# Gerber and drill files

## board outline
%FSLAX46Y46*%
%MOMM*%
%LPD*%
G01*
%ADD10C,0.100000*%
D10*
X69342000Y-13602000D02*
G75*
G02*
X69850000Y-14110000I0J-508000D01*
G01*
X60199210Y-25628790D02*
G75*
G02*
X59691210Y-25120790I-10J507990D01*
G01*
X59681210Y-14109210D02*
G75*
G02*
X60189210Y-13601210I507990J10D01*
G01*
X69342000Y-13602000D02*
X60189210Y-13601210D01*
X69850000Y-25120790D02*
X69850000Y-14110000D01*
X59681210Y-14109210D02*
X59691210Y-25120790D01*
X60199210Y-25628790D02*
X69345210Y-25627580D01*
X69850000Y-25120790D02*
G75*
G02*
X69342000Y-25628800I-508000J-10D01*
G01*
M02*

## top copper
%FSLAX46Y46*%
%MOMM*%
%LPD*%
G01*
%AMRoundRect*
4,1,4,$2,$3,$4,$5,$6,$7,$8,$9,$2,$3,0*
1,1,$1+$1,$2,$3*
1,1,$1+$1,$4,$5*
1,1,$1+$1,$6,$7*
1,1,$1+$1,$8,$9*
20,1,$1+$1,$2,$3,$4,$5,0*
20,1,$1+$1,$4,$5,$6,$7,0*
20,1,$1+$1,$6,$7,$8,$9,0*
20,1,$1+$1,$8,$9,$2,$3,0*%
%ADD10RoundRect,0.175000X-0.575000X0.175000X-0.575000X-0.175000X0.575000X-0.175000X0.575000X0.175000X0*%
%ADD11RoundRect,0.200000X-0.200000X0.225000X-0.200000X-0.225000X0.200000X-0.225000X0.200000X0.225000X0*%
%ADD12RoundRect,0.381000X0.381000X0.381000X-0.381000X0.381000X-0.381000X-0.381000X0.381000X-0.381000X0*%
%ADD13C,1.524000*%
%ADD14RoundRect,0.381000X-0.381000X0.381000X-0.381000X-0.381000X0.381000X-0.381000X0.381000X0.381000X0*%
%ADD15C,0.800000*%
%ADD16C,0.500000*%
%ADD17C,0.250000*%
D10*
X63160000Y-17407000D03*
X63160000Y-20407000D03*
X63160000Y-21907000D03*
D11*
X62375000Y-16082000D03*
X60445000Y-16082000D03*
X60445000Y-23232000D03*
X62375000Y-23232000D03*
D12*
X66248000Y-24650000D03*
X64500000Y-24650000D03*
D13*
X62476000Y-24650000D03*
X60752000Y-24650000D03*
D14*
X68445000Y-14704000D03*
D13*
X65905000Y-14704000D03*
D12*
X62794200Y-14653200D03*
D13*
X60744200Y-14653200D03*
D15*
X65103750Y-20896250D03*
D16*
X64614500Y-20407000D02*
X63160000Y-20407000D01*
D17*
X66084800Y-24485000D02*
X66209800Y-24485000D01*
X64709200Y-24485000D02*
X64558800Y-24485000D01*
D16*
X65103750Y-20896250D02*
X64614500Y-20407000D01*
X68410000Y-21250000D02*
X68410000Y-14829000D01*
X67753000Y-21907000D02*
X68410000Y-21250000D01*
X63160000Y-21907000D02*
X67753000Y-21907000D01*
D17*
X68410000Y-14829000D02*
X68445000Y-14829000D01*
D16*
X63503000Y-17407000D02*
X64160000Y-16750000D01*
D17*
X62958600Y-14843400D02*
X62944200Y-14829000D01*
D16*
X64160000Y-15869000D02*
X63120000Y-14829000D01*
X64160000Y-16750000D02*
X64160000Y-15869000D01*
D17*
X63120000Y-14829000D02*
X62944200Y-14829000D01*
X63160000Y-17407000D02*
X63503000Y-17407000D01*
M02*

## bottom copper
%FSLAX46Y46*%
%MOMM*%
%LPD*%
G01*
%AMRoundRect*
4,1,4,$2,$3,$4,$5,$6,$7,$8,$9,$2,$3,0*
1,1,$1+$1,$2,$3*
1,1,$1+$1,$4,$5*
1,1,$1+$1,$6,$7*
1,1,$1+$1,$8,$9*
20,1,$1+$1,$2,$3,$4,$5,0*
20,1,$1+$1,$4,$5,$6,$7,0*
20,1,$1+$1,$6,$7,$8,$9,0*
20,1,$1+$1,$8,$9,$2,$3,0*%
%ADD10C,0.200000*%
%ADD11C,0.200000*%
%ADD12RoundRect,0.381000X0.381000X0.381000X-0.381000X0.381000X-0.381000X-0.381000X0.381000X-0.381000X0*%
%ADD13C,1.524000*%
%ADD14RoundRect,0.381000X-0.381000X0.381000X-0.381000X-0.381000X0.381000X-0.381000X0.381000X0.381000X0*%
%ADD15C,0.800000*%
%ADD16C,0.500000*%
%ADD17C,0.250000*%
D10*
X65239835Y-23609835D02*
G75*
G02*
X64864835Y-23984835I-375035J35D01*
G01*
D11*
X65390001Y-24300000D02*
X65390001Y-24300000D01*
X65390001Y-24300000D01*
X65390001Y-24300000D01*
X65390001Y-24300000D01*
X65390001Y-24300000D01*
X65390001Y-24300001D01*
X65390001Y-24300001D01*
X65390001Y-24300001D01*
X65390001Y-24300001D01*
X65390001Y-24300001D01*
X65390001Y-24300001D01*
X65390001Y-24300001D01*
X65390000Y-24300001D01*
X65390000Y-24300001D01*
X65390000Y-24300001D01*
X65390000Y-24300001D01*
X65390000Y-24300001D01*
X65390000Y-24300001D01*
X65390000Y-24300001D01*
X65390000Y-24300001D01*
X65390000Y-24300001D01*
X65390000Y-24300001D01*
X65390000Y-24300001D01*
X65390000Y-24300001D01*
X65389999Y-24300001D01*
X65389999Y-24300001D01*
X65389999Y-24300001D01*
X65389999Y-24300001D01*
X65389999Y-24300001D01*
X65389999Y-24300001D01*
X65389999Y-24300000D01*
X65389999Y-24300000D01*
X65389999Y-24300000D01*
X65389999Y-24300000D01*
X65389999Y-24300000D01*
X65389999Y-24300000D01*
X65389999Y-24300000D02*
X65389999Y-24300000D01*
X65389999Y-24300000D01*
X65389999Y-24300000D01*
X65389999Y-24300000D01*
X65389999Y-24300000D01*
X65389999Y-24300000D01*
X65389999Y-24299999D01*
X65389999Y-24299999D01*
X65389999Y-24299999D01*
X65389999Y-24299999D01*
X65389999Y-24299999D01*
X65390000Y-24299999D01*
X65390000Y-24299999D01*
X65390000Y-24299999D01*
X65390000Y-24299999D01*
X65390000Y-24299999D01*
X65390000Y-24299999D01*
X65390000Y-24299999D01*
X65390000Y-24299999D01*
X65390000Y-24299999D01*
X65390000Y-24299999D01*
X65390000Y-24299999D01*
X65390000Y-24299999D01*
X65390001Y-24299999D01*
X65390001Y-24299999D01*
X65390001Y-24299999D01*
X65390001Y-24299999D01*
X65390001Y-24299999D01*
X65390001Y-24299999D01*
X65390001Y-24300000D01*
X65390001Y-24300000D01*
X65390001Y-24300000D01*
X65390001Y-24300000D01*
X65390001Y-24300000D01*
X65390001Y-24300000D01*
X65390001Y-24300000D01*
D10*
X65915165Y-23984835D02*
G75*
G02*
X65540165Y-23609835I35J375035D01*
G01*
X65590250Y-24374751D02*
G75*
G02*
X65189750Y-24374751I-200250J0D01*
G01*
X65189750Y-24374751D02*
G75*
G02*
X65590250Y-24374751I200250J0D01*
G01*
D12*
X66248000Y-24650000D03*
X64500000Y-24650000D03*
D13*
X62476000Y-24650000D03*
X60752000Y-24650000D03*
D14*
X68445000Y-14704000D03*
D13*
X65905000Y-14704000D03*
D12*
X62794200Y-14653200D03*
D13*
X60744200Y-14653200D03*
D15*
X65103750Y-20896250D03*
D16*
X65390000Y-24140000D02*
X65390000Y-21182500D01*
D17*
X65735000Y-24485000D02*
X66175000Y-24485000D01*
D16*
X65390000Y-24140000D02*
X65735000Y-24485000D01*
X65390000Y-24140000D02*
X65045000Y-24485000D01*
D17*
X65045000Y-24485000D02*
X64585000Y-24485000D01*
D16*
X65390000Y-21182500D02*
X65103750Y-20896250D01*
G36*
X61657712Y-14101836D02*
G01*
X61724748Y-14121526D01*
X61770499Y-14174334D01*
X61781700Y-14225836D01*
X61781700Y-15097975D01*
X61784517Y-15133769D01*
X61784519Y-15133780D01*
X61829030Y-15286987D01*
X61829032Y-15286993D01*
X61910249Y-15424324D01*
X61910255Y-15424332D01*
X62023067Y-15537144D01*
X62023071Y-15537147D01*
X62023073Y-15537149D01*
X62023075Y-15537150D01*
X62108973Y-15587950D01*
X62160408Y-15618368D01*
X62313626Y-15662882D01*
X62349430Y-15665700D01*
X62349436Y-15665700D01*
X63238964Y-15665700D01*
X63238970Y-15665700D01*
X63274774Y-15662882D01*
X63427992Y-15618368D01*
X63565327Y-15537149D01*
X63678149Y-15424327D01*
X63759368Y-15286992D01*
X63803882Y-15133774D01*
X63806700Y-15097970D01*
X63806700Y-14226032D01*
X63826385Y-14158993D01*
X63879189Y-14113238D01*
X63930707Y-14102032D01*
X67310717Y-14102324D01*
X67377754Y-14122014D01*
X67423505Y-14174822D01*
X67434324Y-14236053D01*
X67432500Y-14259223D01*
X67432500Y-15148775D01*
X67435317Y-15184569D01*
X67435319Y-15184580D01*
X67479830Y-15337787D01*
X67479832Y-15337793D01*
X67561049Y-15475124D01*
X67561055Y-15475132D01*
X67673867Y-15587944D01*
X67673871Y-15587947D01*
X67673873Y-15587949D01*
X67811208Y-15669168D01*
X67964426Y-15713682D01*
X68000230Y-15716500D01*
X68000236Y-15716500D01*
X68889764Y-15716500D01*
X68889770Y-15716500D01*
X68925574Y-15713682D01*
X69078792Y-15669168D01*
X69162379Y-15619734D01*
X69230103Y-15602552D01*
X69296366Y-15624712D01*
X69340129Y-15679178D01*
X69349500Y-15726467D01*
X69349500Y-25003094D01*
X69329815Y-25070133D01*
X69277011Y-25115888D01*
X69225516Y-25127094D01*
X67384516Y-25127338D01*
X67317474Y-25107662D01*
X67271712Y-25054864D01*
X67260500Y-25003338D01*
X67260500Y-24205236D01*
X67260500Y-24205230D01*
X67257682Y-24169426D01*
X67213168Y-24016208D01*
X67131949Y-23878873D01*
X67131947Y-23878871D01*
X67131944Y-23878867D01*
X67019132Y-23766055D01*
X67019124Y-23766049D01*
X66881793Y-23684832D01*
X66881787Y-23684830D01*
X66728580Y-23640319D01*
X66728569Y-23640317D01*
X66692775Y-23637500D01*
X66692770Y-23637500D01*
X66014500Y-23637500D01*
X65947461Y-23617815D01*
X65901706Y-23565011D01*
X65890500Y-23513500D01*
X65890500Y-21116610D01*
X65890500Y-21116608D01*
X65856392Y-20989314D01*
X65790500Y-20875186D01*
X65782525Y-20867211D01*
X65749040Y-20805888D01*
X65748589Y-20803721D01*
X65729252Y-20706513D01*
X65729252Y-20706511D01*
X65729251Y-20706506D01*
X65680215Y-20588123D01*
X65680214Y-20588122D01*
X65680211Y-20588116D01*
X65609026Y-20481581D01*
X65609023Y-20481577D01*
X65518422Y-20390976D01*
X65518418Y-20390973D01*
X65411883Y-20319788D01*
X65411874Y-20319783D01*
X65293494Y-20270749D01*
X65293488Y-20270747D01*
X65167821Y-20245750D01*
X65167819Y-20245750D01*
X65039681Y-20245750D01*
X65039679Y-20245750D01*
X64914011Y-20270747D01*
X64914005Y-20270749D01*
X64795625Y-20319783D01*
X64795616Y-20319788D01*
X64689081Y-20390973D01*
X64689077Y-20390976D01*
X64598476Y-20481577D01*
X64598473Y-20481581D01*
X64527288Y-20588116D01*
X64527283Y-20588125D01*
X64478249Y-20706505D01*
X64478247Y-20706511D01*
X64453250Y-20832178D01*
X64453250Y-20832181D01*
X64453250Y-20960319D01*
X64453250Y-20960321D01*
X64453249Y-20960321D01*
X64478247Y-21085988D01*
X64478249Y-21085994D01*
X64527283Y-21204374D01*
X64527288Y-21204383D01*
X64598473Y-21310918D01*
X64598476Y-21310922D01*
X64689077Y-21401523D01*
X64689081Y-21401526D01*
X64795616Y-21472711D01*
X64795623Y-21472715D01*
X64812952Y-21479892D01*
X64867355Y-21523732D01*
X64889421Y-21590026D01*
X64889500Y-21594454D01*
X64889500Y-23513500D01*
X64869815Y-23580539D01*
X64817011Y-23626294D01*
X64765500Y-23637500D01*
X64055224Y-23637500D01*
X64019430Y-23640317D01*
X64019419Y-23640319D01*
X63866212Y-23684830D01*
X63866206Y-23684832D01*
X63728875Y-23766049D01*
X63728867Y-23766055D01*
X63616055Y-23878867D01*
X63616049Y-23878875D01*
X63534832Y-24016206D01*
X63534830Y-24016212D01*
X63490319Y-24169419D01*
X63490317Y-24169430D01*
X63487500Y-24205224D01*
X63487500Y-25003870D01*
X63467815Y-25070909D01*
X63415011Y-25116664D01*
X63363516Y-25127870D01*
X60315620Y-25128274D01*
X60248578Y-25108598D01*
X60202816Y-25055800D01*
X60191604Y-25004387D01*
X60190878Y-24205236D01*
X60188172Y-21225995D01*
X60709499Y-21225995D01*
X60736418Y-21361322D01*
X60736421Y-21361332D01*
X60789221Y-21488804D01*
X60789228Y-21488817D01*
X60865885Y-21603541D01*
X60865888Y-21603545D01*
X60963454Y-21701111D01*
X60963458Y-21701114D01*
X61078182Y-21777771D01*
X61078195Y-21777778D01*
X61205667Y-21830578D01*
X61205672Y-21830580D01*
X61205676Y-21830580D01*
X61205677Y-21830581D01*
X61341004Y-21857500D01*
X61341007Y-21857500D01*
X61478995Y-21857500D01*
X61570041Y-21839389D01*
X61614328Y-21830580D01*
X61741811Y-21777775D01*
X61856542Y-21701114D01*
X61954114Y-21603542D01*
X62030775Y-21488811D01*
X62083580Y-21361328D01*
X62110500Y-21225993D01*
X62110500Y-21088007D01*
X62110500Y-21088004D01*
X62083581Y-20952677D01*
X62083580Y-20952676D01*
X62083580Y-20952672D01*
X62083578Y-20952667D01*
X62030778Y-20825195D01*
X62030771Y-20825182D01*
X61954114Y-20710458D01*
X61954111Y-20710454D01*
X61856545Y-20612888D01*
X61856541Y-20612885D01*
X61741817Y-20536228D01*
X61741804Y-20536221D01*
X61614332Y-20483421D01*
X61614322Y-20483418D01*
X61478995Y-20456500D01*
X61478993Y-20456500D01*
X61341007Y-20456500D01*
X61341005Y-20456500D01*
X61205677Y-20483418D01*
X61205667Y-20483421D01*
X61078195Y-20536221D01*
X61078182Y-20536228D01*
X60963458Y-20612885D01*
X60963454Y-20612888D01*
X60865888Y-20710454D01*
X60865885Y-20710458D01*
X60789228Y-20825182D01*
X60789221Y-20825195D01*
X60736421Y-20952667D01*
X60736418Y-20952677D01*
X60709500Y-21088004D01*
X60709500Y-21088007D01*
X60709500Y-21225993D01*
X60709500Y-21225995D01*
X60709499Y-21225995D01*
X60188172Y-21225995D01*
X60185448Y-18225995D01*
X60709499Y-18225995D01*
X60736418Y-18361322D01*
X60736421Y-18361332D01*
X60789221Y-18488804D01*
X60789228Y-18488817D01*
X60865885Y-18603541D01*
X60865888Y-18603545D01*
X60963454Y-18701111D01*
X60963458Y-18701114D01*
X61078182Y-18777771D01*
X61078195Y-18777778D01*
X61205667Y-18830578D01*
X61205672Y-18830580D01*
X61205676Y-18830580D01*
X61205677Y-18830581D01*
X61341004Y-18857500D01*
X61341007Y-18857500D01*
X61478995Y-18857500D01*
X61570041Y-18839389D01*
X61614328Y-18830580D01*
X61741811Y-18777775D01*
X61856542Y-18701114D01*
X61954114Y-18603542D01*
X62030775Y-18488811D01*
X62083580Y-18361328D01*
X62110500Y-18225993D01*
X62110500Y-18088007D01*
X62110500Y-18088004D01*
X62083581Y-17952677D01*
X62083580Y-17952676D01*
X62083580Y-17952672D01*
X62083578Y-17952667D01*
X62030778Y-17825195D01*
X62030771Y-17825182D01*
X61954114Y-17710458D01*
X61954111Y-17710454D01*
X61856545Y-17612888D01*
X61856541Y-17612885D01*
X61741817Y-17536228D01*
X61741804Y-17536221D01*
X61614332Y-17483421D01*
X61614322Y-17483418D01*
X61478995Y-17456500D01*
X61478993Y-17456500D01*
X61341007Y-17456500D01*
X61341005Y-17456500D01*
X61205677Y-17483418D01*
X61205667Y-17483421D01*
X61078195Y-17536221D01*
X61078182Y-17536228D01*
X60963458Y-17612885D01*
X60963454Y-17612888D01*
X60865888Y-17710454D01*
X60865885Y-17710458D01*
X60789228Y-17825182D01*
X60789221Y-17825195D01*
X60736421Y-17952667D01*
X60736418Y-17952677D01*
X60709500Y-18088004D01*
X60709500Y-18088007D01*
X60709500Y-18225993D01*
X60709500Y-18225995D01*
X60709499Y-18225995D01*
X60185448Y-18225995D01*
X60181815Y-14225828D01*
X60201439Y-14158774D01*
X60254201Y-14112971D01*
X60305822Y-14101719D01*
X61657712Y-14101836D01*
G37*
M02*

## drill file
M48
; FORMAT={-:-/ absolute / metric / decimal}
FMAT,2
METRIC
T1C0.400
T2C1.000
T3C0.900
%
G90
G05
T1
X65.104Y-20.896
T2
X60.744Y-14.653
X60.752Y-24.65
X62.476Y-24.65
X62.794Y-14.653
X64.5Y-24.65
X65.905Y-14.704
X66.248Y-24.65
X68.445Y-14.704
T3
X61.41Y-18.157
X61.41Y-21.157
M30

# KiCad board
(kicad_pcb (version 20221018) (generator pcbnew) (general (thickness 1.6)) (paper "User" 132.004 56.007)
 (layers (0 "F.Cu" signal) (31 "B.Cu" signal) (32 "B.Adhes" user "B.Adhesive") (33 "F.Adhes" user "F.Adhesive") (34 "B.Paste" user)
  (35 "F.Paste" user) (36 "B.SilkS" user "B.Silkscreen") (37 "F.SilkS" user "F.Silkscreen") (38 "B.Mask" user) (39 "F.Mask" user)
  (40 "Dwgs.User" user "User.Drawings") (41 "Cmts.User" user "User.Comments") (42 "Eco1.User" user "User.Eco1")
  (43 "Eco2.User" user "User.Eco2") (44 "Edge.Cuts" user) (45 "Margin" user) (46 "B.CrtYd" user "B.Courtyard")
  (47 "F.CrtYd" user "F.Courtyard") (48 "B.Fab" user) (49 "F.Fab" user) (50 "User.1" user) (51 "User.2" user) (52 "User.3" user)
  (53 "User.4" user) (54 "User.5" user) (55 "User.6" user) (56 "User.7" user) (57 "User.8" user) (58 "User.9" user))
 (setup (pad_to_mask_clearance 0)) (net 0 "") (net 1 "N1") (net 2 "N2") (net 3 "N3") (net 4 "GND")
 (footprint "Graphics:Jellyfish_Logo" (layer "F.Cu") (at 68.475 24.4)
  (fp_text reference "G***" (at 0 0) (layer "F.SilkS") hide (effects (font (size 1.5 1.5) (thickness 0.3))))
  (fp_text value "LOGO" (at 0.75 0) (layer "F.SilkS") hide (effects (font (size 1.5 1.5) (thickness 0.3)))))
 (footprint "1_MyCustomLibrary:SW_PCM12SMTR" (layer "F.Cu") (at 61.41 19.657 -90)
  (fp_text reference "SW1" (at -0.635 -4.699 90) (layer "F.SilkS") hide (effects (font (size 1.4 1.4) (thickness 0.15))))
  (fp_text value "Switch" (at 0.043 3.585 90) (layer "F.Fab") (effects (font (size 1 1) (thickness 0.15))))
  (pad "" np_thru_hole circle (at -1.5 0 270) (size 0.9 0.9) (drill 0.9) (layers "*.Cu" "*.Mask"))
  (pad "" np_thru_hole circle (at 1.5 0 270) (size 0.9 0.9) (drill 0.9) (layers "*.Cu" "*.Mask"))
  (pad "1" smd roundrect (at -2.25 -1.75 270) (size 0.7 1.5) (layers "F.Cu" "F.Paste" "F.Mask") (roundrect_rratio 0.25) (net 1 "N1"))
  (pad "2" smd roundrect (at 0.75 -1.75 270) (size 0.7 1.5) (layers "F.Cu" "F.Paste" "F.Mask") (roundrect_rratio 0.25) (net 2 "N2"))
  (pad "3" smd roundrect (at 2.25 -1.75 270) (size 0.7 1.5) (layers "F.Cu" "F.Paste" "F.Mask") (roundrect_rratio 0.25) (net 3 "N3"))
  (pad "S1" smd roundrect (at -3.575 -0.965 270) (size 0.85 0.8) (layers "F.Cu" "F.Paste" "F.Mask") (roundrect_rratio 0.25))
  (pad "S2" smd roundrect (at -3.575 0.965 270) (size 0.85 0.8) (layers "F.Cu" "F.Paste" "F.Mask") (roundrect_rratio 0.25))
  (pad "S3" smd roundrect (at 3.575 0.965 270) (size 0.85 0.8) (layers "F.Cu" "F.Paste" "F.Mask") (roundrect_rratio 0.25))
  (pad "S4" smd roundrect (at 3.575 -0.965 270) (size 0.85 0.8) (layers "F.Cu" "F.Paste" "F.Mask") (roundrect_rratio 0.25)))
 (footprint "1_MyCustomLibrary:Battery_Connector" (layer "F.Cu") (at 64.5 24.65 180)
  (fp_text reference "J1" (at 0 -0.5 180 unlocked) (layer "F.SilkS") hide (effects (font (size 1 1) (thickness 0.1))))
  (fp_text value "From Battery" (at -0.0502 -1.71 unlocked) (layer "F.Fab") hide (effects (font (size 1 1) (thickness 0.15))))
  (pad "1" thru_hole roundrect (at -1.748 0 180) (size 1.524 1.524) (drill oval 1) (layers "*.Cu" "*.Mask") (roundrect_rratio 0.25)
   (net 2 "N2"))
  (pad "1" thru_hole roundrect (at 0 0 180) (size 1.524 1.524) (drill oval 1) (layers "*.Cu" "*.Mask") (roundrect_rratio 0.25) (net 2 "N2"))
  (pad "2" thru_hole circle (at 2.024 0 180) (size 1.524 1.524) (drill 1) (layers "*.Cu" "*.Mask") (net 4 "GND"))
  (pad "2" thru_hole circle (at 3.748 0 180) (size 1.524 1.524) (drill 1) (layers "*.Cu" "*.Mask") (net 4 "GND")))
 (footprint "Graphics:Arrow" (layer "F.Cu") (at 64.8 21.125 180)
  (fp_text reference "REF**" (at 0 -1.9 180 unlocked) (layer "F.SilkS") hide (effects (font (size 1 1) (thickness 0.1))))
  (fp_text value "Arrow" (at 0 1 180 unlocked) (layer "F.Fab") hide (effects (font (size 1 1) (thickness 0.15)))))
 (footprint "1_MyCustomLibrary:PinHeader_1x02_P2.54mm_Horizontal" (layer "F.Cu") (at 68.445 14.704 -90)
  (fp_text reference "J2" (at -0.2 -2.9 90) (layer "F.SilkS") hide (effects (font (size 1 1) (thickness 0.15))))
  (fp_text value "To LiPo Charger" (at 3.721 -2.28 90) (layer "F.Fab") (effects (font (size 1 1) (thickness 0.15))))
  (pad "1" thru_hole roundrect (at 0 0 270) (size 1.524 1.524) (drill 1) (layers "*.Cu" "*.Mask") (roundrect_rratio 0.25) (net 3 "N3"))
  (pad "2" thru_hole circle (at 0 2.54 270) (size 1.524 1.524) (drill 1) (layers "*.Cu" "*.Mask") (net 4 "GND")))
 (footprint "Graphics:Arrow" (layer "F.Cu") (at 64.8 20.615)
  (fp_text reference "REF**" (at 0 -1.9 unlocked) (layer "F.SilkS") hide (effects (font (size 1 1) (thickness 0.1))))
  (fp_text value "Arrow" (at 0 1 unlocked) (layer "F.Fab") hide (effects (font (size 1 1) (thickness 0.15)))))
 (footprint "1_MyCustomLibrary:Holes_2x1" (layer "F.Cu") (at 62.0442 14.6532 180)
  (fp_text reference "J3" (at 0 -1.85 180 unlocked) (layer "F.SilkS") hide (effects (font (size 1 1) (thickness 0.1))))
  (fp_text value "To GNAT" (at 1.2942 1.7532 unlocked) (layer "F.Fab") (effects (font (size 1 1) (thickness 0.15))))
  (pad "1" thru_hole roundrect (at -0.75 0 180) (size 1.524 1.524) (drill 1) (layers "*.Cu" "*.Mask") (roundrect_rratio 0.25) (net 1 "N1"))
  (pad "2" thru_hole circle (at 1.3 0 180) (size 1.524 1.524) (drill 1) (layers "*.Cu" "*.Mask") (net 4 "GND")))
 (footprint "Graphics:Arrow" (layer "B.Cu") (at 60.475 20.05)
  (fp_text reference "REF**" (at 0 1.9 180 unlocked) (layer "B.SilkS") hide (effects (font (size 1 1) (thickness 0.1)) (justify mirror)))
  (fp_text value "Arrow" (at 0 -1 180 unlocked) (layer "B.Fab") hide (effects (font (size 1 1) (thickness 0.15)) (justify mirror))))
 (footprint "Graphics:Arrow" (layer "B.Cu") (at 60.475 19.54 180)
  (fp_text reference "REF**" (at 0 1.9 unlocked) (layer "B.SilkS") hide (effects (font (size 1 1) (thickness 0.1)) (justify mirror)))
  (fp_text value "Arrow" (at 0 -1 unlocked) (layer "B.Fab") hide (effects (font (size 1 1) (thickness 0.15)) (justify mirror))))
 (gr_arc (start 65.239835 23.609835) (mid 65.13 23.875) (end 64.864835 23.984835) (stroke (width 0.2) (type default)) (layer "B.Cu"))
 (gr_circle (center 65.39 24.3) (end 65.39 24.3) (stroke (width 0.2) (type default)) (fill none) (layer "B.Cu"))
 (gr_arc (start 65.915165 23.984835) (mid 65.65 23.875) (end 65.540165 23.609835) (stroke (width 0.2) (type default)) (layer "B.Cu"))
 (gr_circle (center 65.39 24.374751) (end 65.4 24.174751) (stroke (width 0.2) (type default)) (fill none) (layer "B.Cu"))
 (gr_arc (start 69.342 13.602) (mid 69.70121 13.75079) (end 69.85 14.11) (stroke (width 0.1) (type default)) (layer "Edge.Cuts"))
 (gr_arc (start 60.19921 25.62879) (mid 59.84 25.48) (end 59.69121 25.12079) (stroke (width 0.1) (type default)) (layer "Edge.Cuts"))
 (gr_arc (start 59.68121 14.10921) (mid 59.83 13.75) (end 60.18921 13.60121) (stroke (width 0.1) (type default)) (layer "Edge.Cuts"))
 (gr_line (start 69.342 13.602) (end 60.18921 13.60121) (stroke (width 0.1) (type default)) (layer "Edge.Cuts"))
 (gr_line (start 69.85 25.12079) (end 69.85 14.11) (stroke (width 0.1) (type default)) (layer "Edge.Cuts"))
 (gr_line (start 59.68121 14.10921) (end 59.69121 25.12079) (stroke (width 0.1) (type default)) (layer "Edge.Cuts"))
 (gr_line (start 60.19921 25.62879) (end 69.34521 25.62758) (stroke (width 0.1) (type default)) (layer "Edge.Cuts"))
 (gr_arc (start 69.85 25.12079) (mid 69.70121 25.48) (end 69.342 25.62879) (stroke (width 0.1) (type default)) (layer "Edge.Cuts"))
 (segment (start 64.6145 20.407) (end 63.16 20.407) (width 0.5) (layer "F.Cu") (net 2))
 (segment (start 66.0848 24.485) (end 66.2098 24.485) (width 0.25) (layer "F.Cu") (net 2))
 (segment (start 64.7092 24.485) (end 64.5588 24.485) (width 0.25) (layer "F.Cu") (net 2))
 (segment (start 65.10375 20.89625) (end 64.6145 20.407) (width 0.5) (layer "F.Cu") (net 2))
 (via (at 65.10375 20.89625) (size 0.8) (drill 0.4) (layers "F.Cu" "B.Cu") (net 2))
 (segment (start 65.39 24.14) (end 65.39 21.1825) (width 0.5) (layer "B.Cu") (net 2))
 (segment (start 65.735 24.485) (end 66.175 24.485) (width 0.25) (layer "B.Cu") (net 2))
 (segment (start 65.39 24.14) (end 65.735 24.485) (width 0.5) (layer "B.Cu") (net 2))
 (segment (start 65.39 24.14) (end 65.045 24.485) (width 0.5) (layer "B.Cu") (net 2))
 (segment (start 65.045 24.485) (end 64.585 24.485) (width 0.25) (layer "B.Cu") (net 2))
 (segment (start 65.39 21.1825) (end 65.10375 20.89625) (width 0.5) (layer "B.Cu") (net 2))
 (segment (start 68.41 21.25) (end 68.41 14.829) (width 0.5) (layer "F.Cu") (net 3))
 (segment (start 67.753 21.907) (end 68.41 21.25) (width 0.5) (layer "F.Cu") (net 3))
 (segment (start 63.16 21.907) (end 67.753 21.907) (width 0.5) (layer "F.Cu") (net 3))
 (segment (start 68.41 14.829) (end 68.445 14.829) (width 0.25) (layer "F.Cu") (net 3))
 (segment (start 63.503 17.407) (end 64.16 16.75) (width 0.5) (layer "F.Cu") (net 1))
 (segment (start 62.9586 14.8434) (end 62.9442 14.829) (width 0.25) (layer "F.Cu") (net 1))
 (segment (start 64.16 15.869) (end 63.12 14.829) (width 0.5) (layer "F.Cu") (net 1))
 (segment (start 64.16 16.75) (end 64.16 15.869) (width 0.5) (layer "F.Cu") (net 1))
 (segment (start 63.12 14.829) (end 62.9442 14.829) (width 0.25) (layer "F.Cu") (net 1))
 (segment (start 63.16 17.407) (end 63.503 17.407) (width 0.25) (layer "F.Cu") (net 1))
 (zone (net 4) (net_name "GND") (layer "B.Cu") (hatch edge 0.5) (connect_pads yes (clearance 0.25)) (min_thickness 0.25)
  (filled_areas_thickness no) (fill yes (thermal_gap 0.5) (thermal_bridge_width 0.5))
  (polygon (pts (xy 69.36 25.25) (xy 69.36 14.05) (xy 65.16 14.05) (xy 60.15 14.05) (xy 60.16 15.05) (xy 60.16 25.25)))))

